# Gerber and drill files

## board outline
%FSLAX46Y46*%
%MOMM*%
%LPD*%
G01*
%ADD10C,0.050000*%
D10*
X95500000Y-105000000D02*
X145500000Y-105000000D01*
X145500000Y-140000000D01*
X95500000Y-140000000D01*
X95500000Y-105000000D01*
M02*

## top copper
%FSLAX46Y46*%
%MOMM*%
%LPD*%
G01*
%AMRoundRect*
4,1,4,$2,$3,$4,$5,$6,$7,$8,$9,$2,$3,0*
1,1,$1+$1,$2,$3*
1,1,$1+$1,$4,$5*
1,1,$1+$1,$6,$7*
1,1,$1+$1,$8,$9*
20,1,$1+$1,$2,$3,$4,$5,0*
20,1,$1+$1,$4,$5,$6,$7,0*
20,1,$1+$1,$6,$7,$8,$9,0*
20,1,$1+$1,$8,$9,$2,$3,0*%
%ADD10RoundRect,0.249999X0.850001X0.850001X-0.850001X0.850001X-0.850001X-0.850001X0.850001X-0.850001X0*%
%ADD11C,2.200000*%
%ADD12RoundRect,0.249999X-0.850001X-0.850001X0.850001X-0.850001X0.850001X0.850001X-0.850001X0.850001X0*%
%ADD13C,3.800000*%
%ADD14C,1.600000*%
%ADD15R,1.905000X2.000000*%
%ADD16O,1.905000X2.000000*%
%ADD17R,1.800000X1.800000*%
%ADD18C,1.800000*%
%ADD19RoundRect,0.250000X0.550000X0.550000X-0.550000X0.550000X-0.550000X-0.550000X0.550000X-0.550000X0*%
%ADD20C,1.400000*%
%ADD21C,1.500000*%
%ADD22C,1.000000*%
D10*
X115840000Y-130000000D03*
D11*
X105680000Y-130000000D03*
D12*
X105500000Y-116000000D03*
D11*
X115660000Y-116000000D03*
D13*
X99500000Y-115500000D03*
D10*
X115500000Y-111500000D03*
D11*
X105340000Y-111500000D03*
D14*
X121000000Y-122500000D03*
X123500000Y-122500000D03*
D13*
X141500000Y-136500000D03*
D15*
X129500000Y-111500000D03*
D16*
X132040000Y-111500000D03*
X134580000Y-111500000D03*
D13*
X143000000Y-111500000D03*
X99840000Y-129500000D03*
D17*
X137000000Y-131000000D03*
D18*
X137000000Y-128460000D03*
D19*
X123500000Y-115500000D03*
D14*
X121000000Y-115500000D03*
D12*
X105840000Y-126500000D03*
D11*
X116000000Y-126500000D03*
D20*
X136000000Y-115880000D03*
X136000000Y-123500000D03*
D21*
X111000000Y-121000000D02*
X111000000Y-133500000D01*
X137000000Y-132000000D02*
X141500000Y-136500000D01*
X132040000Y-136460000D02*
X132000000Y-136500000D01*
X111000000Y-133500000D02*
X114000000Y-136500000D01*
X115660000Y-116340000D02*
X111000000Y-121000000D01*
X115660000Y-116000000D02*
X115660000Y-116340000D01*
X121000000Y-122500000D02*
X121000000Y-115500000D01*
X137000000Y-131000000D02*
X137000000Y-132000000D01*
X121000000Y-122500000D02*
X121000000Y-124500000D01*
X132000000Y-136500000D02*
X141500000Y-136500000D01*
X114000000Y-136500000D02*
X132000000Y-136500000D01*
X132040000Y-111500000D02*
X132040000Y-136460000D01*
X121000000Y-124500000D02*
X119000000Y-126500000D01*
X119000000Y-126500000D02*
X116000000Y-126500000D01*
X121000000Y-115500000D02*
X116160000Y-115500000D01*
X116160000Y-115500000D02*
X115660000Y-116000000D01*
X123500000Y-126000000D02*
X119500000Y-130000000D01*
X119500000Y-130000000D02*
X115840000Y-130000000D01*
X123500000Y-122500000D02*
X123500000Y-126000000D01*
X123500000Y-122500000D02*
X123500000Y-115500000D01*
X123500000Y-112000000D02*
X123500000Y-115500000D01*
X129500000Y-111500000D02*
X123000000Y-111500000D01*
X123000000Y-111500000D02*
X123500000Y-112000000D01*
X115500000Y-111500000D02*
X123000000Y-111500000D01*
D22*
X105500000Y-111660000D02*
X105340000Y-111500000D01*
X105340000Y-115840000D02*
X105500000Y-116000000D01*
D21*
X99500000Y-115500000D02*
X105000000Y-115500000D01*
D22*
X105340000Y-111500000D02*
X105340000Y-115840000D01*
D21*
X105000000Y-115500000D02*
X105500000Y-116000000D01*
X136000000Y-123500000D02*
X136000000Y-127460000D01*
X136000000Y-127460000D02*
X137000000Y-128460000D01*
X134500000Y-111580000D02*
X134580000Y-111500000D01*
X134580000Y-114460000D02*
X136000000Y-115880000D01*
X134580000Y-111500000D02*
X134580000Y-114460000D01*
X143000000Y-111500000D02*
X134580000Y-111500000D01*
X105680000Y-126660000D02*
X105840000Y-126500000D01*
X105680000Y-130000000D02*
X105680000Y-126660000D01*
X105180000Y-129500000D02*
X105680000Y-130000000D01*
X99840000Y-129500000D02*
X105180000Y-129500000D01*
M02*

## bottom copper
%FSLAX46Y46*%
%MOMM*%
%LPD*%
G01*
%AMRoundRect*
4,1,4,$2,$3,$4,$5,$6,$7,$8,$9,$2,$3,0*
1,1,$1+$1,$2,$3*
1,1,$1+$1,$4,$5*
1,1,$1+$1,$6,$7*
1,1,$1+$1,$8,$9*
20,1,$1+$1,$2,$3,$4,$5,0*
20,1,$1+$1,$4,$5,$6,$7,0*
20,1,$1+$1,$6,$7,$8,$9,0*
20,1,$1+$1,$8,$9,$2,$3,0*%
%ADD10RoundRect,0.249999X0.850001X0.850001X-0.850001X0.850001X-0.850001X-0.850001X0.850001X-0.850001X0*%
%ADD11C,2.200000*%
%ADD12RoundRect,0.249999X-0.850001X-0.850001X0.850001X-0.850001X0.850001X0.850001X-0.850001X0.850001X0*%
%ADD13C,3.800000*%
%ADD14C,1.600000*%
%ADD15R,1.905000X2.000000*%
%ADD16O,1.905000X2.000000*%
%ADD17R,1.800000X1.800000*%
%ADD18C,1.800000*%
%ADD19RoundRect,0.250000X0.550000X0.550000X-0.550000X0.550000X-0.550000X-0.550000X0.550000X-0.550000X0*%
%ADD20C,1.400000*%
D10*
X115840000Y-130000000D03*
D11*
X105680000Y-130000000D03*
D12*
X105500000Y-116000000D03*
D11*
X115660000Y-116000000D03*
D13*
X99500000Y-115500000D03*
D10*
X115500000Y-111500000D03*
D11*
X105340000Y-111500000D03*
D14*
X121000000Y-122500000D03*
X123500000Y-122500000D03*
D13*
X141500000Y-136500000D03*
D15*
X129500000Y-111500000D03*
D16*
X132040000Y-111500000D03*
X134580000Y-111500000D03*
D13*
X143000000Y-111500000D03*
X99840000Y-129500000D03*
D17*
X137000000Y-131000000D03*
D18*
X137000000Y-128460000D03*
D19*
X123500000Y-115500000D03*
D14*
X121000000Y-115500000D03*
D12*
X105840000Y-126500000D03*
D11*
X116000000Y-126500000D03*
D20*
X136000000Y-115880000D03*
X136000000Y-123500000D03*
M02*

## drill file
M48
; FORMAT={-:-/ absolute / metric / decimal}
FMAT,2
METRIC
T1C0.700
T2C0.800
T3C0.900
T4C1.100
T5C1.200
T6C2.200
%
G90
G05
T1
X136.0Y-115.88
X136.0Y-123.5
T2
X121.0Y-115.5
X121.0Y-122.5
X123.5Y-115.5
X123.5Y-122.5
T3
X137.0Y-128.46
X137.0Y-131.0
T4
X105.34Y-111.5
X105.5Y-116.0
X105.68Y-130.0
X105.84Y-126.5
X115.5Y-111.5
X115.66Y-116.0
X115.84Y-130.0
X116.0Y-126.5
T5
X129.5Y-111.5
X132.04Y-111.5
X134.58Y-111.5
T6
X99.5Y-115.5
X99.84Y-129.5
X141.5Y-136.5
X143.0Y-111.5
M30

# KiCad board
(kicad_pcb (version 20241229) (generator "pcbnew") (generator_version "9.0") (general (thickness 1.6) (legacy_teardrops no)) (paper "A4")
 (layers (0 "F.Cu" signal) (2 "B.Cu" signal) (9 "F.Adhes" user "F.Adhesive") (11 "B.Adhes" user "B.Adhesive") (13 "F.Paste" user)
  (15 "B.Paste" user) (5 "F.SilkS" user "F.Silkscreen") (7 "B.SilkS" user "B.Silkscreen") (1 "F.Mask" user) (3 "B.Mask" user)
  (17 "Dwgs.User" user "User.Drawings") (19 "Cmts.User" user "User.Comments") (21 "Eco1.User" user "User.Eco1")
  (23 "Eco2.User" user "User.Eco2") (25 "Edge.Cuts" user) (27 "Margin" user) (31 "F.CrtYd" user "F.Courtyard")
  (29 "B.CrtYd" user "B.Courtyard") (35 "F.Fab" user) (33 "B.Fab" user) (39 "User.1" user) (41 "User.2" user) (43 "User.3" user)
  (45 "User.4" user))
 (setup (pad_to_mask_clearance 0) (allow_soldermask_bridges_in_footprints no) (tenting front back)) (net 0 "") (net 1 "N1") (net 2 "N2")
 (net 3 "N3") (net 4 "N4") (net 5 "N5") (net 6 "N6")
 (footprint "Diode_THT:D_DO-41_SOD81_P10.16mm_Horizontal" (layer "F.Cu") (at 115.84 130 180)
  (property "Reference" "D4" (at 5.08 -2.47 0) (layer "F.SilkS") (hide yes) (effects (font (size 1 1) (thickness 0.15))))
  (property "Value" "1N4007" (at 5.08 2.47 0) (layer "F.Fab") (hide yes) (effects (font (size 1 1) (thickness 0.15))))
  (pad "1" thru_hole roundrect (at 0 0 180) (size 2.2 2.2) (drill 1.1) (layers "*.Cu" "*.Mask") (remove_unused_layers no)
   (roundrect_rratio 0.113636) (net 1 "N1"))
  (pad "2" thru_hole circle (at 10.16 0 180) (size 2.2 2.2) (drill 1.1) (layers "*.Cu" "*.Mask") (remove_unused_layers no) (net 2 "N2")))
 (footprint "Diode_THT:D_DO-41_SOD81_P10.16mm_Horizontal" (layer "F.Cu") (at 105.5 116)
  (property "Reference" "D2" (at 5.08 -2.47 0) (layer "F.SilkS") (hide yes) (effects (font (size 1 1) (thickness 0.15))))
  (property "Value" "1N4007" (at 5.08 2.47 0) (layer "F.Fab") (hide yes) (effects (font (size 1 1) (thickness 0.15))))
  (pad "1" thru_hole roundrect (at 0 0) (size 2.2 2.2) (drill 1.1) (layers "*.Cu" "*.Mask") (remove_unused_layers no)
   (roundrect_rratio 0.113636) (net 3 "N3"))
  (pad "2" thru_hole circle (at 10.16 0) (size 2.2 2.2) (drill 1.1) (layers "*.Cu" "*.Mask") (remove_unused_layers no) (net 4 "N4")))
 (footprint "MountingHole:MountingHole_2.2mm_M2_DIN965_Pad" (layer "F.Cu") (at 99.5 115.5)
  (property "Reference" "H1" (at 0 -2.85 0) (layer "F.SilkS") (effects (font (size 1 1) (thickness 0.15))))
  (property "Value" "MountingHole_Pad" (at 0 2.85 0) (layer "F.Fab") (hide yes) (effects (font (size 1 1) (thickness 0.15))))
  (pad "1" thru_hole circle (at 0 0) (size 3.8 3.8) (drill 2.2) (layers "*.Cu" "*.Mask") (remove_unused_layers no) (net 3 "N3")
   (zone_connect 2)))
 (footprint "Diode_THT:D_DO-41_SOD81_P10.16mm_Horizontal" (layer "F.Cu") (at 115.5 111.5 180)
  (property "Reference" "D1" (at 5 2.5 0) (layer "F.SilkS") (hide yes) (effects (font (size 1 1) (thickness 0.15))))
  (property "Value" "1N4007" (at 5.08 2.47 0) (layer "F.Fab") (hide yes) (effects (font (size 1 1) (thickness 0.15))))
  (pad "1" thru_hole roundrect (at 0 0 180) (size 2.2 2.2) (drill 1.1) (layers "*.Cu" "*.Mask") (remove_unused_layers no)
   (roundrect_rratio 0.113636) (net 1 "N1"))
  (pad "2" thru_hole circle (at 10.16 0 180) (size 2.2 2.2) (drill 1.1) (layers "*.Cu" "*.Mask") (remove_unused_layers no) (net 3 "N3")))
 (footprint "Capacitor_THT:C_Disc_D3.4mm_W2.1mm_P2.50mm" (layer "F.Cu") (at 121 122.5)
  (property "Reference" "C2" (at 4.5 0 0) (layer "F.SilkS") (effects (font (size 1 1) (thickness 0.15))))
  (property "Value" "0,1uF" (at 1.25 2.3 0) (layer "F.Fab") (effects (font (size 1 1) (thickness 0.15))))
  (pad "1" thru_hole circle (at 0 0) (size 1.6 1.6) (drill 0.8) (layers "*.Cu" "*.Mask") (remove_unused_layers no) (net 4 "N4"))
  (pad "2" thru_hole circle (at 2.5 0) (size 1.6 1.6) (drill 0.8) (layers "*.Cu" "*.Mask") (remove_unused_layers no) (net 1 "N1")))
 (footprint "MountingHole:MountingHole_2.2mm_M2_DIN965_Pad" (layer "F.Cu") (at 141.5 136.5)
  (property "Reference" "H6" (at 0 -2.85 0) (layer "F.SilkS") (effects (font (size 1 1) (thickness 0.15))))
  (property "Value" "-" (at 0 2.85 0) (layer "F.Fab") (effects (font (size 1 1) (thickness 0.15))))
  (pad "1" thru_hole circle (at 0 0) (size 3.8 3.8) (drill 2.2) (layers "*.Cu" "*.Mask") (remove_unused_layers no) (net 4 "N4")
   (zone_connect 2)))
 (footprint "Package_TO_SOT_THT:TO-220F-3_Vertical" (layer "F.Cu") (at 129.5 111.5)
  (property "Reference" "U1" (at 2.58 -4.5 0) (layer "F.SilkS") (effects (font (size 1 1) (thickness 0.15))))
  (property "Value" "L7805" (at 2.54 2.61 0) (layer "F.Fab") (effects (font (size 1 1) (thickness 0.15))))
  (pad "1" thru_hole rect (at 0 0) (size 1.905 2) (drill 1.2) (layers "*.Cu" "*.Mask") (remove_unused_layers no) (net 1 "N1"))
  (pad "2" thru_hole oval (at 2.54 0) (size 1.905 2) (drill 1.2) (layers "*.Cu" "*.Mask") (remove_unused_layers no) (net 4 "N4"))
  (pad "3" thru_hole oval (at 5.08 0) (size 1.905 2) (drill 1.2) (layers "*.Cu" "*.Mask") (remove_unused_layers no) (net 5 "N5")))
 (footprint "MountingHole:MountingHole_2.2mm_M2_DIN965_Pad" (layer "F.Cu") (at 143 111.5)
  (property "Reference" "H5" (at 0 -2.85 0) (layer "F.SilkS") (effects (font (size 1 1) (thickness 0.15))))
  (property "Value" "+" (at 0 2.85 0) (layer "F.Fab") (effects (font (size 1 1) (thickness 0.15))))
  (pad "1" thru_hole circle (at 0 0) (size 3.8 3.8) (drill 2.2) (layers "*.Cu" "*.Mask") (remove_unused_layers no) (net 5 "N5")
   (zone_connect 2)))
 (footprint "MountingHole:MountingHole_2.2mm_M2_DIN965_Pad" (layer "F.Cu") (at 99.84 129.5)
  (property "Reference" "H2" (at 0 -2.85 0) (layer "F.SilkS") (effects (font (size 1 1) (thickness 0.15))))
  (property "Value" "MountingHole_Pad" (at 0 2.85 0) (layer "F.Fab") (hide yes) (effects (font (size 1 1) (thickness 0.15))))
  (pad "1" thru_hole circle (at 0 0) (size 3.8 3.8) (drill 2.2) (layers "*.Cu" "*.Mask") (remove_unused_layers no) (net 2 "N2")
   (zone_connect 2)))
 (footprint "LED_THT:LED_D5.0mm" (layer "F.Cu") (at 137 131 90)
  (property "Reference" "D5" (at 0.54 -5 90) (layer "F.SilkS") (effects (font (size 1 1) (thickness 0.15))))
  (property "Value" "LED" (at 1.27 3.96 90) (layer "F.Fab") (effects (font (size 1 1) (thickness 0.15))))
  (pad "1" thru_hole rect (at 0 0 90) (size 1.8 1.8) (drill 0.9) (layers "*.Cu" "*.Mask") (remove_unused_layers no) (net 4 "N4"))
  (pad "2" thru_hole circle (at 2.54 0 90) (size 1.8 1.8) (drill 0.9) (layers "*.Cu" "*.Mask") (remove_unused_layers no) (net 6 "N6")))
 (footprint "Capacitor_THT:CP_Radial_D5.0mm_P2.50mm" (layer "F.Cu") (at 123.5 115.5 180)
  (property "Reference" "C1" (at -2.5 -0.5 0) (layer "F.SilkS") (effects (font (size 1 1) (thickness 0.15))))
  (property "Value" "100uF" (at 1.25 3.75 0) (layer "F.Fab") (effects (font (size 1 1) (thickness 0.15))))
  (pad "1" thru_hole roundrect (at 0 0 180) (size 1.6 1.6) (drill 0.8) (layers "*.Cu" "*.Mask") (remove_unused_layers no)
   (roundrect_rratio 0.15625) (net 1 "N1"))
  (pad "2" thru_hole circle (at 2.5 0 180) (size 1.6 1.6) (drill 0.8) (layers "*.Cu" "*.Mask") (remove_unused_layers no) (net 4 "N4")))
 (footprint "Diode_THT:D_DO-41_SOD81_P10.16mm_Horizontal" (layer "F.Cu") (at 105.84 126.5)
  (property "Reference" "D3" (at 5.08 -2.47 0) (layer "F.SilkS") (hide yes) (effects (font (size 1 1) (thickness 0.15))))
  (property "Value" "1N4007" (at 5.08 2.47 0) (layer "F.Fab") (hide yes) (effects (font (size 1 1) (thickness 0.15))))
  (pad "1" thru_hole roundrect (at 0 0) (size 2.2 2.2) (drill 1.1) (layers "*.Cu" "*.Mask") (remove_unused_layers no)
   (roundrect_rratio 0.113636) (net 2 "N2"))
  (pad "2" thru_hole circle (at 10.16 0) (size 2.2 2.2) (drill 1.1) (layers "*.Cu" "*.Mask") (remove_unused_layers no) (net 4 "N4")))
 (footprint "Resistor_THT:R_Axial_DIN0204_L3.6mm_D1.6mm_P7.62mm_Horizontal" (layer "F.Cu") (at 136 115.88 -90)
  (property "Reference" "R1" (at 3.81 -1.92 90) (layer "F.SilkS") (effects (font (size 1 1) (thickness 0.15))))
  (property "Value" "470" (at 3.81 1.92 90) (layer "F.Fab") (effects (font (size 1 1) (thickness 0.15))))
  (pad "1" thru_hole circle (at 0 0 270) (size 1.4 1.4) (drill 0.7) (layers "*.Cu" "*.Mask") (remove_unused_layers no) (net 5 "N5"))
  (pad "2" thru_hole circle (at 7.62 0 270) (size 1.4 1.4) (drill 0.7) (layers "*.Cu" "*.Mask") (remove_unused_layers no) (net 6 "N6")))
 (gr_rect (start 95.5 105) (end 145.5 140) (stroke (width 0.05) (type default)) (fill no) (layer "Edge.Cuts"))
 (segment (start 111 121) (end 111 133.5) (width 1.5) (layer "F.Cu") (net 4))
 (segment (start 137 132) (end 141.5 136.5) (width 1.5) (layer "F.Cu") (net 4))
 (segment (start 132.04 136.46) (end 132 136.5) (width 1.5) (layer "F.Cu") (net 4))
 (segment (start 111 133.5) (end 114 136.5) (width 1.5) (layer "F.Cu") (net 4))
 (segment (start 115.66 116.34) (end 111 121) (width 1.5) (layer "F.Cu") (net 4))
 (segment (start 115.66 116) (end 115.66 116.34) (width 1.5) (layer "F.Cu") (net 4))
 (segment (start 121 122.5) (end 121 115.5) (width 1.5) (layer "F.Cu") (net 4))
 (segment (start 137 131) (end 137 132) (width 1.5) (layer "F.Cu") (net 4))
 (segment (start 121 122.5) (end 121 124.5) (width 1.5) (layer "F.Cu") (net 4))
 (segment (start 132 136.5) (end 141.5 136.5) (width 1.5) (layer "F.Cu") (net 4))
 (segment (start 114 136.5) (end 132 136.5) (width 1.5) (layer "F.Cu") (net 4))
 (segment (start 132.04 111.5) (end 132.04 136.46) (width 1.5) (layer "F.Cu") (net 4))
 (segment (start 121 124.5) (end 119 126.5) (width 1.5) (layer "F.Cu") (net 4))
 (segment (start 119 126.5) (end 116 126.5) (width 1.5) (layer "F.Cu") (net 4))
 (segment (start 121 115.5) (end 116.16 115.5) (width 1.5) (layer "F.Cu") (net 4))
 (segment (start 116.16 115.5) (end 115.66 116) (width 1.5) (layer "F.Cu") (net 4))
 (segment (start 123.5 126) (end 119.5 130) (width 1.5) (layer "F.Cu") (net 1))
 (segment (start 119.5 130) (end 115.84 130) (width 1.5) (layer "F.Cu") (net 1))
 (segment (start 123.5 122.5) (end 123.5 126) (width 1.5) (layer "F.Cu") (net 1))
 (segment (start 123.5 122.5) (end 123.5 115.5) (width 1.5) (layer "F.Cu") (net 1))
 (segment (start 123.5 112) (end 123.5 115.5) (width 1.5) (layer "F.Cu") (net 1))
 (segment (start 129.5 111.5) (end 123 111.5) (width 1.5) (layer "F.Cu") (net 1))
 (segment (start 123 111.5) (end 123.5 112) (width 1.5) (layer "F.Cu") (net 1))
 (segment (start 115.5 111.5) (end 123 111.5) (width 1.5) (layer "F.Cu") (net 1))
 (segment (start 105.5 111.66) (end 105.34 111.5) (width 1) (layer "F.Cu") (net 3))
 (segment (start 105.34 115.84) (end 105.5 116) (width 1) (layer "F.Cu") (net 3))
 (segment (start 99.5 115.5) (end 105 115.5) (width 1.5) (layer "F.Cu") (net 3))
 (segment (start 105.34 111.5) (end 105.34 115.84) (width 1) (layer "F.Cu") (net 3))
 (segment (start 105 115.5) (end 105.5 116) (width 1.5) (layer "F.Cu") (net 3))
 (segment (start 136 123.5) (end 136 127.46) (width 1.5) (layer "F.Cu") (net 6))
 (segment (start 136 127.46) (end 137 128.46) (width 1.5) (layer "F.Cu") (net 6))
 (segment (start 134.5 111.58) (end 134.58 111.5) (width 1.5) (layer "F.Cu") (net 5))
 (segment (start 134.58 114.46) (end 136 115.88) (width 1.5) (layer "F.Cu") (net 5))
 (segment (start 134.58 111.5) (end 134.58 114.46) (width 1.5) (layer "F.Cu") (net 5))
 (segment (start 143 111.5) (end 134.58 111.5) (width 1.5) (layer "F.Cu") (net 5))
 (segment (start 105.68 126.66) (end 105.84 126.5) (width 1.5) (layer "F.Cu") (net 2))
 (segment (start 105.68 130) (end 105.68 126.66) (width 1.5) (layer "F.Cu") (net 2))
 (segment (start 105.18 129.5) (end 105.68 130) (width 1.5) (layer "F.Cu") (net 2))
 (segment (start 99.84 129.5) (end 105.18 129.5) (width 1.5) (layer "F.Cu") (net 2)))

